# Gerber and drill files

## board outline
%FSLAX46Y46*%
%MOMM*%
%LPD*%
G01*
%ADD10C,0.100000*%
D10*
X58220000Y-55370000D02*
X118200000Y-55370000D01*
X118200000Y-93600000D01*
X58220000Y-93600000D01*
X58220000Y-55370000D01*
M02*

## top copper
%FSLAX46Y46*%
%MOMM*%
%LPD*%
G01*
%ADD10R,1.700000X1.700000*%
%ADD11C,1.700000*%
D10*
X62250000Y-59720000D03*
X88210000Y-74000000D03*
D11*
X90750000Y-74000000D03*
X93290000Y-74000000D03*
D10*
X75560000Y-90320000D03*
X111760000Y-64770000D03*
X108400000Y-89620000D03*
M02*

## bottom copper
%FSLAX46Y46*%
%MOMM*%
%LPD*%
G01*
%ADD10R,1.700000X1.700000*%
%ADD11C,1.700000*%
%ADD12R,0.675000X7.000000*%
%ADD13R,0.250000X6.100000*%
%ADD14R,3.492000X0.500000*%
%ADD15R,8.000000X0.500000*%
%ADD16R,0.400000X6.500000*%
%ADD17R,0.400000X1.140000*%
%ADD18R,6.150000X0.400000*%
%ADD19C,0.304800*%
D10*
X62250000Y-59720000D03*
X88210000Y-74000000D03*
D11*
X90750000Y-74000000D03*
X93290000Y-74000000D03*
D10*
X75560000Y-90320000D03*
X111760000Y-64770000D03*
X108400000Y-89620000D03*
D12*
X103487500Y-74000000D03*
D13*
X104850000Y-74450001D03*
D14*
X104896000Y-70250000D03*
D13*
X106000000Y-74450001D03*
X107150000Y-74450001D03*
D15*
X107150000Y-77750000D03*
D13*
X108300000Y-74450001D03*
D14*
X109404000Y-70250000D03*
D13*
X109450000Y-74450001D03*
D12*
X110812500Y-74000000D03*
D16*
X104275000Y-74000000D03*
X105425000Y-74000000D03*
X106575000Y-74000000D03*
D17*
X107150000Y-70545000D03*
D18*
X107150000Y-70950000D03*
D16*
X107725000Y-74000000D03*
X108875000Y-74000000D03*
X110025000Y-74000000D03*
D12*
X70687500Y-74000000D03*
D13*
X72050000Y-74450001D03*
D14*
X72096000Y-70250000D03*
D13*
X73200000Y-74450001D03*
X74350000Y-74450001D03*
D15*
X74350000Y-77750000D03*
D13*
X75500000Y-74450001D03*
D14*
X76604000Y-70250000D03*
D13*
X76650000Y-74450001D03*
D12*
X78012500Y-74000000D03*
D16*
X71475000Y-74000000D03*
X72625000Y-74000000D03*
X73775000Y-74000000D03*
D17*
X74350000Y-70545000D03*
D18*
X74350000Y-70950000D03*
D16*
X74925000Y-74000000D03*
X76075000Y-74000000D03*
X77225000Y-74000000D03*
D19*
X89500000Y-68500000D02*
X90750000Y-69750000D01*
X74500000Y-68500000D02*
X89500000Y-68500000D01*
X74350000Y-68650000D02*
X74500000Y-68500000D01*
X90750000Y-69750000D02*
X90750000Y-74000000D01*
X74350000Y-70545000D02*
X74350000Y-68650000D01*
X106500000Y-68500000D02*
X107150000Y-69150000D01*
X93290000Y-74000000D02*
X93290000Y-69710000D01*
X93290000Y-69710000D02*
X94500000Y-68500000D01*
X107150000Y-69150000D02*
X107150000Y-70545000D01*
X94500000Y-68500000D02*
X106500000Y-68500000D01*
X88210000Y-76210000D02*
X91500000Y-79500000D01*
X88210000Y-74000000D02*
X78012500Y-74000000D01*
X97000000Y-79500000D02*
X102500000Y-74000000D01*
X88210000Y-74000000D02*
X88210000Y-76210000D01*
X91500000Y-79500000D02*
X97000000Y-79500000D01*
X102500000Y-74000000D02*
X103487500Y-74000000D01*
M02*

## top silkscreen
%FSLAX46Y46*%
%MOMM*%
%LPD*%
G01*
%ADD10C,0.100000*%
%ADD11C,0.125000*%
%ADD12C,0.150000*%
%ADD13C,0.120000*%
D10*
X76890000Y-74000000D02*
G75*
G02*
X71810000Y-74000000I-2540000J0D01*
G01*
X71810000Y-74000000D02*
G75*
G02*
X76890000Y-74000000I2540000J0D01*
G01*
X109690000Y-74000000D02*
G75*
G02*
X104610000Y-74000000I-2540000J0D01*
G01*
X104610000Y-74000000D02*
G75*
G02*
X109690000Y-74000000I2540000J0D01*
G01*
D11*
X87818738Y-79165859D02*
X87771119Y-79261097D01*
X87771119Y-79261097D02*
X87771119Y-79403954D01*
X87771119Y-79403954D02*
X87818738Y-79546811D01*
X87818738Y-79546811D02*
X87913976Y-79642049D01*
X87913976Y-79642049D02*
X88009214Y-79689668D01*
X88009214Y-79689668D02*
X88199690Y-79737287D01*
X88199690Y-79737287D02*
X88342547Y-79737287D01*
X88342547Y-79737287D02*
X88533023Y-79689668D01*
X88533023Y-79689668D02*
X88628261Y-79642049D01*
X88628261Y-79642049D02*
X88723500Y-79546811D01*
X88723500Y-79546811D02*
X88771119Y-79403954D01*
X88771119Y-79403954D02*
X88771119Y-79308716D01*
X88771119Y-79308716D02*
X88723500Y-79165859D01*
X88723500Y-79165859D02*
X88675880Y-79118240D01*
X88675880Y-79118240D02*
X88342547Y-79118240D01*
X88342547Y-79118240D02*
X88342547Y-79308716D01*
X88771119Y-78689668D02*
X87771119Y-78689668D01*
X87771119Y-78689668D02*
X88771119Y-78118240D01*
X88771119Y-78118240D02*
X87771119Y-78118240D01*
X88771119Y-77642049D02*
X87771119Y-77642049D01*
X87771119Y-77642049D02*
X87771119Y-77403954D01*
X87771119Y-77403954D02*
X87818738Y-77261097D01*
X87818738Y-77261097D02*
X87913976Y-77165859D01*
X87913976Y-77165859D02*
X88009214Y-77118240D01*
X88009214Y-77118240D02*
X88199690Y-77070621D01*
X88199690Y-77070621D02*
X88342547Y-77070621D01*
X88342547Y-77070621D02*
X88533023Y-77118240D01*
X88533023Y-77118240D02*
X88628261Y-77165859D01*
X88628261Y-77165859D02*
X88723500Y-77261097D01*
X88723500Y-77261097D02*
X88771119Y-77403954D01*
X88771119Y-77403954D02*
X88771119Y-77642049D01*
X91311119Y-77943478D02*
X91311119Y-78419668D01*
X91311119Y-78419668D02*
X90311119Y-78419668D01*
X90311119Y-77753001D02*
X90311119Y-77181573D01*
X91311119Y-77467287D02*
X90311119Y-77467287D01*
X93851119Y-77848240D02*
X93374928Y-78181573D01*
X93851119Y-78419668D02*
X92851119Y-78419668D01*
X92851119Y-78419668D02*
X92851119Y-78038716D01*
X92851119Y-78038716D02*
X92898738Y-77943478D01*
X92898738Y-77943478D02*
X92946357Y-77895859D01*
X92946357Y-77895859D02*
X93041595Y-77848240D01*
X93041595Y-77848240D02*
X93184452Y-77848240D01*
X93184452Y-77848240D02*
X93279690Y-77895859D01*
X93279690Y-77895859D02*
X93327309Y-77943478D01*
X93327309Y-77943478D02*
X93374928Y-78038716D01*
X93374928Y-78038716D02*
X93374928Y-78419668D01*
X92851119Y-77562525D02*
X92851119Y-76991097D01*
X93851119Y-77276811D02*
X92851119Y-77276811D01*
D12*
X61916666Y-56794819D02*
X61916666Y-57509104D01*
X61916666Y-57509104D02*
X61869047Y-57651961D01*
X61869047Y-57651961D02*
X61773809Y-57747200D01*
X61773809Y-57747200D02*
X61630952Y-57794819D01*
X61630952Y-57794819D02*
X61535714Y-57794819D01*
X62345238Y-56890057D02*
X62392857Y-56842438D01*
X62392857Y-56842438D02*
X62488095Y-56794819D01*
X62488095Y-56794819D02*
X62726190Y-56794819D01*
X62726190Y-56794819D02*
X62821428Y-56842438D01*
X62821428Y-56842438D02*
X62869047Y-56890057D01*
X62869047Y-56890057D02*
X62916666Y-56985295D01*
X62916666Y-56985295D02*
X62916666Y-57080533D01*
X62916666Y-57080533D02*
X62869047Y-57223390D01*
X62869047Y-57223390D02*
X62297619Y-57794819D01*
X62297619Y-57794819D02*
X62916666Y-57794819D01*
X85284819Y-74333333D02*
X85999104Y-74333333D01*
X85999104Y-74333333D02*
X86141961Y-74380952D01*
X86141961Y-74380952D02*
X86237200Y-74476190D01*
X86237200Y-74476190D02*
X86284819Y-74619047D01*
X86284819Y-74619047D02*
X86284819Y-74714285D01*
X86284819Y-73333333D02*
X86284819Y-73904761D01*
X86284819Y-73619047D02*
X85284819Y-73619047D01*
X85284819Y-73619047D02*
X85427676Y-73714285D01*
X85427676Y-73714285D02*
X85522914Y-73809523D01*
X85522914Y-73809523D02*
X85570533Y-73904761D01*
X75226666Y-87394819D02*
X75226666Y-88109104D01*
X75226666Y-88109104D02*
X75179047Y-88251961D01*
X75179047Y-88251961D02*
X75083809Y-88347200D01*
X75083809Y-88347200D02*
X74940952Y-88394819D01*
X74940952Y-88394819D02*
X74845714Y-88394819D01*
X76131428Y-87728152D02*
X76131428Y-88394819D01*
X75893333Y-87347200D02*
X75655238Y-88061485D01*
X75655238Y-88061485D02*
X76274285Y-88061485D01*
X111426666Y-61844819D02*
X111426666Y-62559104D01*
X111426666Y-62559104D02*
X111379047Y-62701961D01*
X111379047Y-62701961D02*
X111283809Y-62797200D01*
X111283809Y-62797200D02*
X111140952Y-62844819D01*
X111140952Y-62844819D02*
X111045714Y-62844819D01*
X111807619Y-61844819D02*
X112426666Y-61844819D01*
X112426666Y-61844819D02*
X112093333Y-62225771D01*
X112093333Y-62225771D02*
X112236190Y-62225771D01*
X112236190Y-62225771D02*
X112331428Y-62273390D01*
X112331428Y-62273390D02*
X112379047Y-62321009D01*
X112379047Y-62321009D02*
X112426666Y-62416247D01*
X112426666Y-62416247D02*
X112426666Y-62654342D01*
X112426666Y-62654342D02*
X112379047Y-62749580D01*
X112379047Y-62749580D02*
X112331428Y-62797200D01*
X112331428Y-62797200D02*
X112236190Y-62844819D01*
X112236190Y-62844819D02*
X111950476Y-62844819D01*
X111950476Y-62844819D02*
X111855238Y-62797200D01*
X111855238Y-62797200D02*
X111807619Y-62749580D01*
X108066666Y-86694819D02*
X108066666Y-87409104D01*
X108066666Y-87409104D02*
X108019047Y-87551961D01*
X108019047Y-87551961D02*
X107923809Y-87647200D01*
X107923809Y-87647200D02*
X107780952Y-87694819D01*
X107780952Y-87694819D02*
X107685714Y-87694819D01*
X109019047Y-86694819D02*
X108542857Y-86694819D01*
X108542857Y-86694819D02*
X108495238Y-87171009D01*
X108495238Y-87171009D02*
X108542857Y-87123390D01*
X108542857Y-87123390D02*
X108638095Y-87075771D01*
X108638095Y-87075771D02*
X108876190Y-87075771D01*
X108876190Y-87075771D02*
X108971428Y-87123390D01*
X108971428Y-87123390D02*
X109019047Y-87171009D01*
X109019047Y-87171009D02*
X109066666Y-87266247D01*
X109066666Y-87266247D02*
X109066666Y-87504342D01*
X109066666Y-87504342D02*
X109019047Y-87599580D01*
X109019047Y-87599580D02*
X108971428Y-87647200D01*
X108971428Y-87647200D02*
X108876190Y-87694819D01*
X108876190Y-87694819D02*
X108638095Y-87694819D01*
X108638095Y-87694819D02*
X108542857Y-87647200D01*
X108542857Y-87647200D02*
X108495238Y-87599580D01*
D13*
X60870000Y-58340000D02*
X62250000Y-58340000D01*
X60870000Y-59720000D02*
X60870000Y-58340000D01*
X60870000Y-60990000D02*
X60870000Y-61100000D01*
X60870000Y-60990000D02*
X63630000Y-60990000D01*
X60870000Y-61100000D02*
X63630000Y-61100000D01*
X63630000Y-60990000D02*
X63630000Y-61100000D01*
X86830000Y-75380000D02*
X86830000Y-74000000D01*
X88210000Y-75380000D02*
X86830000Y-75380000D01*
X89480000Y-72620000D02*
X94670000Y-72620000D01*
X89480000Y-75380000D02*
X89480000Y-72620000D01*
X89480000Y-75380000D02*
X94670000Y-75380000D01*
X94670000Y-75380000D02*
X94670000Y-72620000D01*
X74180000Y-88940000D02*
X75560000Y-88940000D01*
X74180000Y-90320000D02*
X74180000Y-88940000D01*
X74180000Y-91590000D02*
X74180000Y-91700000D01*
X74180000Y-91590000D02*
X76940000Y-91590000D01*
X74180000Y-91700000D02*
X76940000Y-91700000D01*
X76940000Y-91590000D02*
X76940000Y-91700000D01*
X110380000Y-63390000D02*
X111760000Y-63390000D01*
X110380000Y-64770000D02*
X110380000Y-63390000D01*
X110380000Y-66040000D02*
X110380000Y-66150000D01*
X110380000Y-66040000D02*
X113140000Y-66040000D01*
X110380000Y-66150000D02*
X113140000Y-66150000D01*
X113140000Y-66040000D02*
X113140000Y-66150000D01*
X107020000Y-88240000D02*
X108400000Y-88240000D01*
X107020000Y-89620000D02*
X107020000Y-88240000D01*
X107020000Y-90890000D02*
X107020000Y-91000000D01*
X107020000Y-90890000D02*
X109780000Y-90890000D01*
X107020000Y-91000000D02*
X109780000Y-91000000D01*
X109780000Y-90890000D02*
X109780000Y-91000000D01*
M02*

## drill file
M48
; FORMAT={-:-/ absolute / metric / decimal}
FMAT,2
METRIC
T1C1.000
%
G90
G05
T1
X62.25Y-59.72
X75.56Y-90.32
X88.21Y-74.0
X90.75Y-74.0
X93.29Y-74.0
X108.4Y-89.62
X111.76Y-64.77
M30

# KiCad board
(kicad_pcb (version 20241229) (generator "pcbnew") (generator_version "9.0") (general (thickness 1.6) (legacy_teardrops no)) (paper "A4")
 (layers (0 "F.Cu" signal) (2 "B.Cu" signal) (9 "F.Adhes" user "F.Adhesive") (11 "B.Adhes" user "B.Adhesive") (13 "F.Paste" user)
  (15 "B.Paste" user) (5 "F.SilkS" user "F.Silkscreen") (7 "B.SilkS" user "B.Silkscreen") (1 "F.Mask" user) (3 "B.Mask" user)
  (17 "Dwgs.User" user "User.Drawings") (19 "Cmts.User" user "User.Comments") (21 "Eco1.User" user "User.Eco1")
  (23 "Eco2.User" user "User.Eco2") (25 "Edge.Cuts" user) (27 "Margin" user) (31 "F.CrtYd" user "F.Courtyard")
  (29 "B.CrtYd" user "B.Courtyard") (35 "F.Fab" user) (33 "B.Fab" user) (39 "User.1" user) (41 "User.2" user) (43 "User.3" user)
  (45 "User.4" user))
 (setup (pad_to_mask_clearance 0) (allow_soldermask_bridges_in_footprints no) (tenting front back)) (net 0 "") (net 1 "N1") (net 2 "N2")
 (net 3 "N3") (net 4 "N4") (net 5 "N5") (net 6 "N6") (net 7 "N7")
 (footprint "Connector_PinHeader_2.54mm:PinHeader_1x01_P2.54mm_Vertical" (layer "F.Cu") (at 62.25 59.72)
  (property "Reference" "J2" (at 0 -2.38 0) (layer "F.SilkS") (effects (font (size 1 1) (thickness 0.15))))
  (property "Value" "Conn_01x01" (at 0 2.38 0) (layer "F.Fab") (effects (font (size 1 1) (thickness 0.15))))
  (fp_line (start -1.38 -1.38) (end 0 -1.38) (stroke (width 0.12) (type solid)) (layer "F.SilkS"))
  (fp_line (start -1.38 0) (end -1.38 -1.38) (stroke (width 0.12) (type solid)) (layer "F.SilkS"))
  (fp_line (start -1.38 1.27) (end -1.38 1.38) (stroke (width 0.12) (type solid)) (layer "F.SilkS"))
  (fp_line (start -1.38 1.27) (end 1.38 1.27) (stroke (width 0.12) (type solid)) (layer "F.SilkS"))
  (fp_line (start -1.38 1.38) (end 1.38 1.38) (stroke (width 0.12) (type solid)) (layer "F.SilkS"))
  (fp_line (start 1.38 1.27) (end 1.38 1.38) (stroke (width 0.12) (type solid)) (layer "F.SilkS"))
  (pad "1" thru_hole rect (at 0 0) (size 1.7 1.7) (drill 1) (layers "*.Cu" "*.Mask") (remove_unused_layers no) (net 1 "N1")))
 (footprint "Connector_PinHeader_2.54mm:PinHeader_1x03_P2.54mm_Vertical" (layer "F.Cu") (at 88.21 74 90)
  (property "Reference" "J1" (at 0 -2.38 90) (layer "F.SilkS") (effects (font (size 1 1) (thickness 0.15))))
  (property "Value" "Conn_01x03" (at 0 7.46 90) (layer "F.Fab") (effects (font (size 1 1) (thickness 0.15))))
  (fp_line (start -1.38 -1.38) (end 0 -1.38) (stroke (width 0.12) (type solid)) (layer "F.SilkS"))
  (fp_line (start -1.38 0) (end -1.38 -1.38) (stroke (width 0.12) (type solid)) (layer "F.SilkS"))
  (fp_line (start 1.38 1.27) (end 1.38 6.46) (stroke (width 0.12) (type solid)) (layer "F.SilkS"))
  (fp_line (start -1.38 1.27) (end 1.38 1.27) (stroke (width 0.12) (type solid)) (layer "F.SilkS"))
  (fp_line (start -1.38 1.27) (end -1.38 6.46) (stroke (width 0.12) (type solid)) (layer "F.SilkS"))
  (fp_line (start -1.38 6.46) (end 1.38 6.46) (stroke (width 0.12) (type solid)) (layer "F.SilkS"))
  (pad "1" thru_hole rect (at 0 0 90) (size 1.7 1.7) (drill 1) (layers "*.Cu" "*.Mask") (remove_unused_layers no) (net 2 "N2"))
  (pad "2" thru_hole circle (at 0 2.54 90) (size 1.7 1.7) (drill 1) (layers "*.Cu" "*.Mask") (remove_unused_layers no) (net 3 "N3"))
  (pad "3" thru_hole circle (at 0 5.08 90) (size 1.7 1.7) (drill 1) (layers "*.Cu" "*.Mask") (remove_unused_layers no) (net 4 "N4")))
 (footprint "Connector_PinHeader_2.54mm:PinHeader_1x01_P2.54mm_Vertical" (layer "F.Cu") (at 75.56 90.32)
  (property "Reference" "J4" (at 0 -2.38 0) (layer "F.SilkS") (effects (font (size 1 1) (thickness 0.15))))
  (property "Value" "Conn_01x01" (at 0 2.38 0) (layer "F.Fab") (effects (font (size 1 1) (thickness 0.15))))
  (fp_line (start -1.38 -1.38) (end 0 -1.38) (stroke (width 0.12) (type solid)) (layer "F.SilkS"))
  (fp_line (start -1.38 0) (end -1.38 -1.38) (stroke (width 0.12) (type solid)) (layer "F.SilkS"))
  (fp_line (start -1.38 1.27) (end -1.38 1.38) (stroke (width 0.12) (type solid)) (layer "F.SilkS"))
  (fp_line (start -1.38 1.27) (end 1.38 1.27) (stroke (width 0.12) (type solid)) (layer "F.SilkS"))
  (fp_line (start -1.38 1.38) (end 1.38 1.38) (stroke (width 0.12) (type solid)) (layer "F.SilkS"))
  (fp_line (start 1.38 1.27) (end 1.38 1.38) (stroke (width 0.12) (type solid)) (layer "F.SilkS"))
  (pad "1" thru_hole rect (at 0 0) (size 1.7 1.7) (drill 1) (layers "*.Cu" "*.Mask") (remove_unused_layers no) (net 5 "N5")))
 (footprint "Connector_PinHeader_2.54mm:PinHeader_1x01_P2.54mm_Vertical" (layer "F.Cu") (at 111.76 64.77)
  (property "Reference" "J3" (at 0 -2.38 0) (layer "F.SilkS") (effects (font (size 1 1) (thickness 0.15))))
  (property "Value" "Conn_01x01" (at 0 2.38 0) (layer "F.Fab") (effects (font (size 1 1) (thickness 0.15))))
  (fp_line (start -1.38 -1.38) (end 0 -1.38) (stroke (width 0.12) (type solid)) (layer "F.SilkS"))
  (fp_line (start -1.38 0) (end -1.38 -1.38) (stroke (width 0.12) (type solid)) (layer "F.SilkS"))
  (fp_line (start -1.38 1.27) (end -1.38 1.38) (stroke (width 0.12) (type solid)) (layer "F.SilkS"))
  (fp_line (start -1.38 1.27) (end 1.38 1.27) (stroke (width 0.12) (type solid)) (layer "F.SilkS"))
  (fp_line (start -1.38 1.38) (end 1.38 1.38) (stroke (width 0.12) (type solid)) (layer "F.SilkS"))
  (fp_line (start 1.38 1.27) (end 1.38 1.38) (stroke (width 0.12) (type solid)) (layer "F.SilkS"))
  (pad "1" thru_hole rect (at 0 0) (size 1.7 1.7) (drill 1) (layers "*.Cu" "*.Mask") (remove_unused_layers no) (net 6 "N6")))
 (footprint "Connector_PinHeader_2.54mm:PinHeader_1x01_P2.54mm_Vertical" (layer "F.Cu") (at 108.4 89.62)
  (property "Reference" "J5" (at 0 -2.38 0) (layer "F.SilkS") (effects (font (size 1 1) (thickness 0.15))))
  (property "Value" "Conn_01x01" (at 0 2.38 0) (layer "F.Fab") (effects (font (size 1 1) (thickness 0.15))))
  (fp_line (start -1.38 -1.38) (end 0 -1.38) (stroke (width 0.12) (type solid)) (layer "F.SilkS"))
  (fp_line (start -1.38 0) (end -1.38 -1.38) (stroke (width 0.12) (type solid)) (layer "F.SilkS"))
  (fp_line (start -1.38 1.27) (end -1.38 1.38) (stroke (width 0.12) (type solid)) (layer "F.SilkS"))
  (fp_line (start -1.38 1.27) (end 1.38 1.27) (stroke (width 0.12) (type solid)) (layer "F.SilkS"))
  (fp_line (start -1.38 1.38) (end 1.38 1.38) (stroke (width 0.12) (type solid)) (layer "F.SilkS"))
  (fp_line (start 1.38 1.27) (end 1.38 1.38) (stroke (width 0.12) (type solid)) (layer "F.SilkS"))
  (pad "1" thru_hole rect (at 0 0) (size 1.7 1.7) (drill 1) (layers "*.Cu" "*.Mask") (remove_unused_layers no) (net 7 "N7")))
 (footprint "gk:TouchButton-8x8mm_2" (layer "B.Cu") (at 107.15 74)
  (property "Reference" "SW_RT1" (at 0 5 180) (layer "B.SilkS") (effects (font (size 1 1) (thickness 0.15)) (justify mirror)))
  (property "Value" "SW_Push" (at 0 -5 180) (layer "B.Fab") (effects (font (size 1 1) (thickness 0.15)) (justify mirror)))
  (pad "1" smd rect (at -3.6625 0) (size 0.675 7) (layers "B.Cu") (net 2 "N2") (zone_connect 2) (thermal_bridge_angle 45))
  (pad "1" smd rect (at -2.3 0.450001) (size 0.25 6.1) (layers "B.Cu") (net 2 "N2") (zone_connect 2) (thermal_bridge_angle 45))
  (pad "1" smd rect (at -2.254 -3.75) (size 3.492 0.5) (layers "B.Cu") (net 2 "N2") (zone_connect 2) (thermal_bridge_angle 45))
  (pad "1" smd rect (at -1.15 0.450001) (size 0.25 6.1) (layers "B.Cu") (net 2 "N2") (zone_connect 2) (thermal_bridge_angle 45))
  (pad "1" smd rect (at 0 0.450001) (size 0.25 6.1) (layers "B.Cu") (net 2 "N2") (zone_connect 2) (thermal_bridge_angle 45))
  (pad "1" smd rect (at 0 3.75) (size 8 0.5) (layers "B.Cu") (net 2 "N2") (zone_connect 2) (thermal_bridge_angle 45))
  (pad "1" smd rect (at 1.15 0.450001) (size 0.25 6.1) (layers "B.Cu") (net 2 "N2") (zone_connect 2) (thermal_bridge_angle 45))
  (pad "1" smd rect (at 2.254 -3.75) (size 3.492 0.5) (layers "B.Cu") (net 2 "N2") (zone_connect 2) (thermal_bridge_angle 45))
  (pad "1" smd rect (at 2.3 0.450001) (size 0.25 6.1) (layers "B.Cu") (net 2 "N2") (zone_connect 2) (thermal_bridge_angle 45))
  (pad "1" smd rect (at 3.6625 0) (size 0.675 7) (layers "B.Cu") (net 2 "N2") (zone_connect 2) (thermal_bridge_angle 45))
  (pad "2" smd rect (at -2.875 0) (size 0.4 6.5) (layers "B.Cu") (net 4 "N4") (zone_connect 2) (thermal_bridge_angle 45))
  (pad "2" smd rect (at -1.725 0) (size 0.4 6.5) (layers "B.Cu") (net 4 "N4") (zone_connect 2) (thermal_bridge_angle 45))
  (pad "2" smd rect (at -0.575 0) (size 0.4 6.5) (layers "B.Cu") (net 4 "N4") (zone_connect 2) (thermal_bridge_angle 45))
  (pad "2" smd rect (at 0 -3.455) (size 0.4 1.14) (layers "B.Cu") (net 4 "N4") (zone_connect 2) (thermal_bridge_angle 45))
  (pad "2" smd rect (at 0 -3.05) (size 6.15 0.4) (layers "B.Cu") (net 4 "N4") (zone_connect 2) (thermal_bridge_angle 45))
  (pad "2" smd rect (at 0.575 0) (size 0.4 6.5) (layers "B.Cu") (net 4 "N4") (zone_connect 2) (thermal_bridge_angle 45))
  (pad "2" smd rect (at 1.725 0) (size 0.4 6.5) (layers "B.Cu") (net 4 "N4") (zone_connect 2) (thermal_bridge_angle 45))
  (pad "2" smd rect (at 2.875 0) (size 0.4 6.5) (layers "B.Cu") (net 4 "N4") (zone_connect 2) (thermal_bridge_angle 45)))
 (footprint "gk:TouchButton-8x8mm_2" (layer "B.Cu") (at 74.35 74)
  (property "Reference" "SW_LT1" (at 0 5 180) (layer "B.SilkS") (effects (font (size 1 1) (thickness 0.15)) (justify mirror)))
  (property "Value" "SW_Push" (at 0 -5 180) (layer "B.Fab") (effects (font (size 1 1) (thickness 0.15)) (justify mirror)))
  (pad "1" smd rect (at -3.6625 0) (size 0.675 7) (layers "B.Cu") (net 2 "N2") (zone_connect 2) (thermal_bridge_angle 45))
  (pad "1" smd rect (at -2.3 0.450001) (size 0.25 6.1) (layers "B.Cu") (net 2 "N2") (zone_connect 2) (thermal_bridge_angle 45))
  (pad "1" smd rect (at -2.254 -3.75) (size 3.492 0.5) (layers "B.Cu") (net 2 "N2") (zone_connect 2) (thermal_bridge_angle 45))
  (pad "1" smd rect (at -1.15 0.450001) (size 0.25 6.1) (layers "B.Cu") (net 2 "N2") (zone_connect 2) (thermal_bridge_angle 45))
  (pad "1" smd rect (at 0 0.450001) (size 0.25 6.1) (layers "B.Cu") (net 2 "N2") (zone_connect 2) (thermal_bridge_angle 45))
  (pad "1" smd rect (at 0 3.75) (size 8 0.5) (layers "B.Cu") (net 2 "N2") (zone_connect 2) (thermal_bridge_angle 45))
  (pad "1" smd rect (at 1.15 0.450001) (size 0.25 6.1) (layers "B.Cu") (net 2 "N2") (zone_connect 2) (thermal_bridge_angle 45))
  (pad "1" smd rect (at 2.254 -3.75) (size 3.492 0.5) (layers "B.Cu") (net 2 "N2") (zone_connect 2) (thermal_bridge_angle 45))
  (pad "1" smd rect (at 2.3 0.450001) (size 0.25 6.1) (layers "B.Cu") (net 2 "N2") (zone_connect 2) (thermal_bridge_angle 45))
  (pad "1" smd rect (at 3.6625 0) (size 0.675 7) (layers "B.Cu") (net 2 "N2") (zone_connect 2) (thermal_bridge_angle 45))
  (pad "2" smd rect (at -2.875 0) (size 0.4 6.5) (layers "B.Cu") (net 3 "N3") (zone_connect 2) (thermal_bridge_angle 45))
  (pad "2" smd rect (at -1.725 0) (size 0.4 6.5) (layers "B.Cu") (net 3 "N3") (zone_connect 2) (thermal_bridge_angle 45))
  (pad "2" smd rect (at -0.575 0) (size 0.4 6.5) (layers "B.Cu") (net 3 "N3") (zone_connect 2) (thermal_bridge_angle 45))
  (pad "2" smd rect (at 0 -3.455) (size 0.4 1.14) (layers "B.Cu") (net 3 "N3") (zone_connect 2) (thermal_bridge_angle 45))
  (pad "2" smd rect (at 0 -3.05) (size 6.15 0.4) (layers "B.Cu") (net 3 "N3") (zone_connect 2) (thermal_bridge_angle 45))
  (pad "2" smd rect (at 0.575 0) (size 0.4 6.5) (layers "B.Cu") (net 3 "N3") (zone_connect 2) (thermal_bridge_angle 45))
  (pad "2" smd rect (at 1.725 0) (size 0.4 6.5) (layers "B.Cu") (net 3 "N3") (zone_connect 2) (thermal_bridge_angle 45))
  (pad "2" smd rect (at 2.875 0) (size 0.4 6.5) (layers "B.Cu") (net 3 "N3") (zone_connect 2) (thermal_bridge_angle 45)))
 (gr_circle (center 74.35 74) (end 76.89 74) (stroke (width 0.1) (type default)) (fill no) (layer "F.SilkS"))
 (gr_circle (center 107.15 74) (end 109.69 74) (stroke (width 0.1) (type default)) (fill no) (layer "F.SilkS"))
 (gr_rect (start 58.22 55.37) (end 118.2 93.6) (stroke (width 0.1) (type default)) (fill no) (layer "Edge.Cuts"))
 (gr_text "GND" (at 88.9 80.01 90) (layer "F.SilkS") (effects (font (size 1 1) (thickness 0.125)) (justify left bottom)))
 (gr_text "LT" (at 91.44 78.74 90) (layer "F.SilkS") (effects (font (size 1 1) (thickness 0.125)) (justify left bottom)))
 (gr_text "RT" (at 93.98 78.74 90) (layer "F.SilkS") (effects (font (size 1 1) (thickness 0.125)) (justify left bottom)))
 (segment (start 89.5 68.5) (end 90.75 69.75) (width 0.3048) (layer "B.Cu") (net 3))
 (segment (start 74.5 68.5) (end 89.5 68.5) (width 0.3048) (layer "B.Cu") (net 3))
 (segment (start 74.35 68.65) (end 74.5 68.5) (width 0.3048) (layer "B.Cu") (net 3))
 (segment (start 90.75 69.75) (end 90.75 74) (width 0.3048) (layer "B.Cu") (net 3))
 (segment (start 74.35 70.545) (end 74.35 68.65) (width 0.3048) (layer "B.Cu") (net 3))
 (segment (start 106.5 68.5) (end 107.15 69.15) (width 0.3048) (layer "B.Cu") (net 4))
 (segment (start 93.29 74) (end 93.29 69.71) (width 0.3048) (layer "B.Cu") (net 4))
 (segment (start 93.29 69.71) (end 94.5 68.5) (width 0.3048) (layer "B.Cu") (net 4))
 (segment (start 107.15 69.15) (end 107.15 70.545) (width 0.3048) (layer "B.Cu") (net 4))
 (segment (start 94.5 68.5) (end 106.5 68.5) (width 0.3048) (layer "B.Cu") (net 4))
 (segment (start 88.21 76.21) (end 91.5 79.5) (width 0.3048) (layer "B.Cu") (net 2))
 (segment (start 88.21 74) (end 78.0125 74) (width 0.3048) (layer "B.Cu") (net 2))
 (segment (start 97 79.5) (end 102.5 74) (width 0.3048) (layer "B.Cu") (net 2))
 (segment (start 88.21 74) (end 88.21 76.21) (width 0.3048) (layer "B.Cu") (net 2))
 (segment (start 91.5 79.5) (end 97 79.5) (width 0.3048) (layer "B.Cu") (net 2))
 (segment (start 102.5 74) (end 103.4875 74) (width 0.3048) (layer "B.Cu") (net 2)))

